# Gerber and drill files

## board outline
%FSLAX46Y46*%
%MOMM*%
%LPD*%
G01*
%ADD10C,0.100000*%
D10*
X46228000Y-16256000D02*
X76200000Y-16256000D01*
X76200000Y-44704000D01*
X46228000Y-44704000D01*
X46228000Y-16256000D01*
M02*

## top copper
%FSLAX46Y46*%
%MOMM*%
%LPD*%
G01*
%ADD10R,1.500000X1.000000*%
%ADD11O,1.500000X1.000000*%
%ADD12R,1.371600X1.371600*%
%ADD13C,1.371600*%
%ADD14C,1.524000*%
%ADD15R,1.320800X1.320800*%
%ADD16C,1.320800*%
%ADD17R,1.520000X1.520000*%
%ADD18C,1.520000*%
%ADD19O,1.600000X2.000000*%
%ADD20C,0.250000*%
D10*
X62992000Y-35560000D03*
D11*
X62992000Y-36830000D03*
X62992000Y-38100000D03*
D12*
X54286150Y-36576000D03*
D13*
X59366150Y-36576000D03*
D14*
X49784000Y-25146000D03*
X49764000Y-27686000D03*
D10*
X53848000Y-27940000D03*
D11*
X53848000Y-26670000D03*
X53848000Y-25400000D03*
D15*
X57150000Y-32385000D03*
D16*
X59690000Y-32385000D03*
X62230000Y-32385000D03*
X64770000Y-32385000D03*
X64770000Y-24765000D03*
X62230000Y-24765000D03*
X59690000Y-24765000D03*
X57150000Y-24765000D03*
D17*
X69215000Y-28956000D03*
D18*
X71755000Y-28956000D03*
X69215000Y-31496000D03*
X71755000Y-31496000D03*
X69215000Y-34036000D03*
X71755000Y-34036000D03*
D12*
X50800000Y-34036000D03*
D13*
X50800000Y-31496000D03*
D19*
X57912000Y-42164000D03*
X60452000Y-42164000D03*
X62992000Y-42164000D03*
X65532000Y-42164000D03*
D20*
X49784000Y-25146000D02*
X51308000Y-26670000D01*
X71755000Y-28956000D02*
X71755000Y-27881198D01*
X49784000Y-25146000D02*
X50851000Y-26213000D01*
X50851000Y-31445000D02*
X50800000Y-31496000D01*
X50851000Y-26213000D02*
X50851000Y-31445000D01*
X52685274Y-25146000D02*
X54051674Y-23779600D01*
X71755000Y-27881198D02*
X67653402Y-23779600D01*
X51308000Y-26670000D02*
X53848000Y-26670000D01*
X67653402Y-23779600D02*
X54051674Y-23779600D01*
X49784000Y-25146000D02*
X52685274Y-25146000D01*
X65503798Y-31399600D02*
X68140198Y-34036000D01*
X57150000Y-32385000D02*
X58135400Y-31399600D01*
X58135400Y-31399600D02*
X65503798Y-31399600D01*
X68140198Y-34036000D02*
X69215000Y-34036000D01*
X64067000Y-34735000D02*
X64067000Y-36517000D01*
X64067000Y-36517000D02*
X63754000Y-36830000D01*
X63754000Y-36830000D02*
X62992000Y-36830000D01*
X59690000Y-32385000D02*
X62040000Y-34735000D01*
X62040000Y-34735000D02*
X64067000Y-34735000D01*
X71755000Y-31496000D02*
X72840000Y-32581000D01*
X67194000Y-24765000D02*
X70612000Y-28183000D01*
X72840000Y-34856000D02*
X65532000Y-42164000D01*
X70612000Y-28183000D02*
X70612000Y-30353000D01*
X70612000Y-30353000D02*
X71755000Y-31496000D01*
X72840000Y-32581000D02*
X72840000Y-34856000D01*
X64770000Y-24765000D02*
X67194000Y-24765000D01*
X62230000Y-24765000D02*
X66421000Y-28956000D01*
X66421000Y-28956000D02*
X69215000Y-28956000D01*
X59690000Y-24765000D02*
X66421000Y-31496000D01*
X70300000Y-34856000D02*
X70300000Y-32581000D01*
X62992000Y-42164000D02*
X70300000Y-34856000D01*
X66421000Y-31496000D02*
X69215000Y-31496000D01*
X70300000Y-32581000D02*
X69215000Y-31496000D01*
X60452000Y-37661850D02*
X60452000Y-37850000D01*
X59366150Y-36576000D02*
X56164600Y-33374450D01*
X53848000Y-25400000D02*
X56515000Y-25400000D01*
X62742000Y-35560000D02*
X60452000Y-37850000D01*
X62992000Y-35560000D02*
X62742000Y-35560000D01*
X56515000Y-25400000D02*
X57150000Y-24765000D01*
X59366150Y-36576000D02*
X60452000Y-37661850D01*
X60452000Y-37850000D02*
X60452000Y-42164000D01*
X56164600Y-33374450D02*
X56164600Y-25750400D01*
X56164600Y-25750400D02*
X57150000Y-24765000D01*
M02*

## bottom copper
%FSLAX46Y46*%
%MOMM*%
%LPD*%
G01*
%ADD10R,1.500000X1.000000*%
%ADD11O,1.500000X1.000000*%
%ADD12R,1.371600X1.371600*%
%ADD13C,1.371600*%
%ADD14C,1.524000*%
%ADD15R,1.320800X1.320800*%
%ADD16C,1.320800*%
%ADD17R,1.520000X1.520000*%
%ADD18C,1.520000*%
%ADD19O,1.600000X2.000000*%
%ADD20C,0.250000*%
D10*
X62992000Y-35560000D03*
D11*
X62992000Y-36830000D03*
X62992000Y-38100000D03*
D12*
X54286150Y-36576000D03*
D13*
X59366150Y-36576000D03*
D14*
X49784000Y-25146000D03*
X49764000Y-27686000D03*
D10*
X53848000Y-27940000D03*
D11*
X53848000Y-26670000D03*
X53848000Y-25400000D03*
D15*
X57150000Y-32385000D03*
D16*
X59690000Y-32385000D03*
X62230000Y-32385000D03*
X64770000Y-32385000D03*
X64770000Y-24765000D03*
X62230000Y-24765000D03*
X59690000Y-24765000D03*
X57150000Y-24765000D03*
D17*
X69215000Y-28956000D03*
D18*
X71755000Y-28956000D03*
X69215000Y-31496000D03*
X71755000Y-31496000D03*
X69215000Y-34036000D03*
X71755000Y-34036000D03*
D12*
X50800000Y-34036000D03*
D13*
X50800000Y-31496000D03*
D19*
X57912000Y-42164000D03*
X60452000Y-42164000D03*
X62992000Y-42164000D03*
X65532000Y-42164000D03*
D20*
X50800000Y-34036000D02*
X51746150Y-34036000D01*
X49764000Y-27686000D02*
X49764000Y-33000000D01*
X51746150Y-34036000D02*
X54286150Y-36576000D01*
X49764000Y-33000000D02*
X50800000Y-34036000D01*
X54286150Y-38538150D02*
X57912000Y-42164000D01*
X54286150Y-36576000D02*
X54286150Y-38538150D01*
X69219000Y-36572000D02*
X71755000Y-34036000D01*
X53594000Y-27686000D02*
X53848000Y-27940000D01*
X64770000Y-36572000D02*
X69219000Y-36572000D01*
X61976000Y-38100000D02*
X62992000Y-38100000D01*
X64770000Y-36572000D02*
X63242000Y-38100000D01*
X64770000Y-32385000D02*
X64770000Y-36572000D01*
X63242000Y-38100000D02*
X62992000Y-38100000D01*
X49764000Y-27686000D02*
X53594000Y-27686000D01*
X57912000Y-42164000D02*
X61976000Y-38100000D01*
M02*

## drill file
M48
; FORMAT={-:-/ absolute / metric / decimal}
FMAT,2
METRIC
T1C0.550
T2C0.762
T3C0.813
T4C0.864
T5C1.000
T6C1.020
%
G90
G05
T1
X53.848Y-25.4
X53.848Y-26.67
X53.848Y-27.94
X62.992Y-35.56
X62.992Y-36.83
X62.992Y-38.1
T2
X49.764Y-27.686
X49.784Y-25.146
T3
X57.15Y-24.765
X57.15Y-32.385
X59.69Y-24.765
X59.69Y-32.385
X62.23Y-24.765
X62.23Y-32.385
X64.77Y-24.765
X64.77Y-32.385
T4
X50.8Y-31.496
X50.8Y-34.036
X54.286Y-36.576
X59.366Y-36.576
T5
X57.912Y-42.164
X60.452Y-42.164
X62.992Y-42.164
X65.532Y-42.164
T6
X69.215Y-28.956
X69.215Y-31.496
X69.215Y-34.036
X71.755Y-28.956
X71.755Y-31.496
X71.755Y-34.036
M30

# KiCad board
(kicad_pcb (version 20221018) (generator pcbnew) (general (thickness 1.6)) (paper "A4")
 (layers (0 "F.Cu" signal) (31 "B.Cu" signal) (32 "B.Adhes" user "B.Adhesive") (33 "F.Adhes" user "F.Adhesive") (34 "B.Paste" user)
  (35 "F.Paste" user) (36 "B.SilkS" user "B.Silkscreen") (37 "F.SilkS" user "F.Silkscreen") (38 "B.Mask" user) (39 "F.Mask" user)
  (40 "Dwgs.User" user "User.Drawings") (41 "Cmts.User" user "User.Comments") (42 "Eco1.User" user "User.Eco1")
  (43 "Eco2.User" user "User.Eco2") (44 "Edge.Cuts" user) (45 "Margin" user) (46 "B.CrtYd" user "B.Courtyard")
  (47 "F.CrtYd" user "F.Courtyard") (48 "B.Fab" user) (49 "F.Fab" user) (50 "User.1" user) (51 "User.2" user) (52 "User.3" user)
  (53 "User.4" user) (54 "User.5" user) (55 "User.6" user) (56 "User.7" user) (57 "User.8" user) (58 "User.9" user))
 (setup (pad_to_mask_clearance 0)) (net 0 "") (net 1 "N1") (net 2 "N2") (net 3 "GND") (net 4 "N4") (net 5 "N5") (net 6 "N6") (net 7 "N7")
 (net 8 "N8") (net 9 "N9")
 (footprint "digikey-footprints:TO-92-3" (layer "F.Cu") (at 62.992 35.56 -90)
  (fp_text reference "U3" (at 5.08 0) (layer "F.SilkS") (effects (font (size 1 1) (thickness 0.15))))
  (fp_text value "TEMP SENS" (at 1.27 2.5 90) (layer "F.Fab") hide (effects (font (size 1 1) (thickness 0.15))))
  (pad "1" thru_hole rect (at 0 0 90) (size 1 1.5) (drill 0.55) (layers "*.Cu" "*.Mask") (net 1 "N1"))
  (pad "2" thru_hole oval (at 1.27 0 90) (size 1 1.5) (drill 0.55) (layers "*.Cu" "*.Mask") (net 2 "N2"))
  (pad "3" thru_hole oval (at 2.54 0 90) (size 1 1.5) (drill 0.55) (layers "*.Cu" "*.Mask") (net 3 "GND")))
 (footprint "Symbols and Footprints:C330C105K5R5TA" (layer "F.Cu") (at 54.28615 36.576)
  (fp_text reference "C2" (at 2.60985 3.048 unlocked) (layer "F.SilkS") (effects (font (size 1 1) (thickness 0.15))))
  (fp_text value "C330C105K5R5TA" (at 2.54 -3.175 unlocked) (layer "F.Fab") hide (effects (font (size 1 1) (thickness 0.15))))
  (pad "1" thru_hole rect (at 0 0) (size 1.3716 1.3716) (drill 0.8636) (layers "*.Cu" "*.Mask") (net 3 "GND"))
  (pad "2" thru_hole circle (at 5.08 0) (size 1.3716 1.3716) (drill 0.8636) (layers "*.Cu" "*.Mask") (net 1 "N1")))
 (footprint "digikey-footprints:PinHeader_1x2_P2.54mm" (layer "F.Cu") (at 49.784 25.146 -90)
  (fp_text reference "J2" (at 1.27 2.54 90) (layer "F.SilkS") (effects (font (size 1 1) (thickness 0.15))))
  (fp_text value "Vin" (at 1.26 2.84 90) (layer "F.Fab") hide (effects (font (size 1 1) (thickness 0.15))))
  (pad "1" thru_hole circle (at 0 0 270) (size 1.524 1.524) (drill 0.762) (layers "*.Cu" "*.Mask") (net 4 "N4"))
  (pad "2" thru_hole circle (at 2.54 0.02 270) (size 1.524 1.524) (drill 0.762) (layers "*.Cu" "*.Mask") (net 3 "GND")))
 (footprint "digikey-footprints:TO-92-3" (layer "F.Cu") (at 53.848 27.94 90)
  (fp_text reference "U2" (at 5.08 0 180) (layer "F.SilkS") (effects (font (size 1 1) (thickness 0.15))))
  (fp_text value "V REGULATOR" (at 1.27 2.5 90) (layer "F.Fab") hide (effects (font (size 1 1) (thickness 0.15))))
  (pad "1" thru_hole rect (at 0 0 270) (size 1 1.5) (drill 0.55) (layers "*.Cu" "*.Mask") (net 3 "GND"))
  (pad "2" thru_hole oval (at 1.27 0 270) (size 1 1.5) (drill 0.55) (layers "*.Cu" "*.Mask") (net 4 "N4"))
  (pad "3" thru_hole oval (at 2.54 0 270) (size 1 1.5) (drill 0.55) (layers "*.Cu" "*.Mask") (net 1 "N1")))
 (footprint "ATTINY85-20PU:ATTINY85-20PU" (layer "F.Cu") (at 60.96 28.575 90)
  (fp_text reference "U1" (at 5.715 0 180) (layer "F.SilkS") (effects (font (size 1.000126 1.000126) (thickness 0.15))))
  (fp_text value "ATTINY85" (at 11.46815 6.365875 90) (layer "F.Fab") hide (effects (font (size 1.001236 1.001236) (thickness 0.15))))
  (pad "1" thru_hole rect (at -3.81 -3.81 90) (size 1.3208 1.3208) (drill 0.8128) (layers "*.Cu" "*.Mask") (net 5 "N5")
   (solder_mask_margin 0.102))
  (pad "2" thru_hole circle (at -3.81 -1.27 90) (size 1.3208 1.3208) (drill 0.8128) (layers "*.Cu" "*.Mask") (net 2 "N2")
   (solder_mask_margin 0.102))
  (pad "3" thru_hole circle (at -3.81 1.27 90) (size 1.3208 1.3208) (drill 0.8128) (layers "*.Cu" "*.Mask") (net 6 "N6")
   (solder_mask_margin 0.102))
  (pad "4" thru_hole circle (at -3.81 3.81 90) (size 1.3208 1.3208) (drill 0.8128) (layers "*.Cu" "*.Mask") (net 3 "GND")
   (solder_mask_margin 0.102))
  (pad "5" thru_hole circle (at 3.81 3.81 90) (size 1.3208 1.3208) (drill 0.8128) (layers "*.Cu" "*.Mask") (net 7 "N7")
   (solder_mask_margin 0.102))
  (pad "6" thru_hole circle (at 3.81 1.27 90) (size 1.3208 1.3208) (drill 0.8128) (layers "*.Cu" "*.Mask") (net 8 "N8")
   (solder_mask_margin 0.102))
  (pad "7" thru_hole circle (at 3.81 -1.27 90) (size 1.3208 1.3208) (drill 0.8128) (layers "*.Cu" "*.Mask") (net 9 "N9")
   (solder_mask_margin 0.102))
  (pad "8" thru_hole circle (at 3.81 -3.81 90) (size 1.3208 1.3208) (drill 0.8128) (layers "*.Cu" "*.Mask") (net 1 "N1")
   (solder_mask_margin 0.102)))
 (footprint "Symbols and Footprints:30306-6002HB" (layer "F.Cu") (at 69.215 28.956)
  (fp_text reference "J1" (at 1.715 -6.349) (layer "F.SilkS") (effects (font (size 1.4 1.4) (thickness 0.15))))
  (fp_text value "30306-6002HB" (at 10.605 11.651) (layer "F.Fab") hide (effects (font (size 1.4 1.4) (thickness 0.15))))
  (pad "1" thru_hole rect (at 0 0) (size 1.52 1.52) (drill 1.02) (layers "*.Cu" "*.Mask") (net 8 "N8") (solder_mask_margin 0.102))
  (pad "2" thru_hole circle (at 2.54 0) (size 1.52 1.52) (drill 1.02) (layers "*.Cu" "*.Mask") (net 4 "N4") (solder_mask_margin 0.102))
  (pad "3" thru_hole circle (at 0 2.54) (size 1.52 1.52) (drill 1.02) (layers "*.Cu" "*.Mask") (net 9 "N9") (solder_mask_margin 0.102))
  (pad "4" thru_hole circle (at 2.54 2.54) (size 1.52 1.52) (drill 1.02) (layers "*.Cu" "*.Mask") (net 7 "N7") (solder_mask_margin 0.102))
  (pad "5" thru_hole circle (at 0 5.08) (size 1.52 1.52) (drill 1.02) (layers "*.Cu" "*.Mask") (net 5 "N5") (solder_mask_margin 0.102))
  (pad "6" thru_hole circle (at 2.54 5.08) (size 1.52 1.52) (drill 1.02) (layers "*.Cu" "*.Mask") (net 3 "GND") (solder_mask_margin 0.102)))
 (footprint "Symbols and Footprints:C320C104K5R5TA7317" (layer "F.Cu") (at 50.8 34.036 90)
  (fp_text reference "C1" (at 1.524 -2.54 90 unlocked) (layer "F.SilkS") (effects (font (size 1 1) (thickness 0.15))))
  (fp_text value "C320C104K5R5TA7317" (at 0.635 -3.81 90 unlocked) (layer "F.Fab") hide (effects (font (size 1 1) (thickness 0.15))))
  (pad "1" thru_hole rect (at 0 0 90) (size 1.3716 1.3716) (drill 0.8636) (layers "*.Cu" "*.Mask") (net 3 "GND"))
  (pad "2" thru_hole circle (at 2.54 0 90) (size 1.3716 1.3716) (drill 0.8636) (layers "*.Cu" "*.Mask") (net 4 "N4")))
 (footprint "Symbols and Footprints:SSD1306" (layer "B.Cu") (at 61.532 31.564)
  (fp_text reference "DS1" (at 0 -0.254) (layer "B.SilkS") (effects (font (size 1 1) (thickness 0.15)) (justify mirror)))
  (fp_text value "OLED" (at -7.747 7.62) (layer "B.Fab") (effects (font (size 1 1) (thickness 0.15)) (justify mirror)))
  (pad "1" thru_hole oval (at -3.62 10.6 270) (size 2 1.6) (drill 1) (layers "*.Cu" "*.Mask") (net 3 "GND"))
  (pad "2" thru_hole oval (at -1.08 10.6 270) (size 2 1.6) (drill 1) (layers "*.Cu" "*.Mask") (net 1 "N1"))
  (pad "3" thru_hole oval (at 1.46 10.6 270) (size 2 1.6) (drill 1) (layers "*.Cu" "*.Mask") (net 9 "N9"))
  (pad "4" thru_hole oval (at 4 10.6 270) (size 2 1.6) (drill 1) (layers "*.Cu" "*.Mask") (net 7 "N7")))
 (gr_rect (start 46.228 16.256) (end 76.2 44.704) (stroke (width 0.1) (type default)) (fill none) (layer "Edge.Cuts"))
 (segment (start 49.784 25.146) (end 51.308 26.67) (width 0.25) (layer "F.Cu") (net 4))
 (segment (start 71.755 28.956) (end 71.755 27.881198) (width 0.25) (layer "F.Cu") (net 4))
 (segment (start 49.784 25.146) (end 50.851 26.213) (width 0.25) (layer "F.Cu") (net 4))
 (segment (start 50.851 31.445) (end 50.8 31.496) (width 0.25) (layer "F.Cu") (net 4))
 (segment (start 50.851 26.213) (end 50.851 31.445) (width 0.25) (layer "F.Cu") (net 4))
 (segment (start 52.685274 25.146) (end 54.051674 23.7796) (width 0.25) (layer "F.Cu") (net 4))
 (segment (start 71.755 27.881198) (end 67.653402 23.7796) (width 0.25) (layer "F.Cu") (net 4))
 (segment (start 51.308 26.67) (end 53.848 26.67) (width 0.25) (layer "F.Cu") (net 4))
 (segment (start 67.653402 23.7796) (end 54.051674 23.7796) (width 0.25) (layer "F.Cu") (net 4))
 (segment (start 49.784 25.146) (end 52.685274 25.146) (width 0.25) (layer "F.Cu") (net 4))
 (segment (start 50.8 34.036) (end 51.74615 34.036) (width 0.25) (layer "B.Cu") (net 3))
 (segment (start 49.764 27.686) (end 49.764 33) (width 0.25) (layer "B.Cu") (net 3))
 (segment (start 51.74615 34.036) (end 54.28615 36.576) (width 0.25) (layer "B.Cu") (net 3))
 (segment (start 49.764 33) (end 50.8 34.036) (width 0.25) (layer "B.Cu") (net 3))
 (segment (start 54.28615 38.53815) (end 57.912 42.164) (width 0.25) (layer "B.Cu") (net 3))
 (segment (start 54.28615 36.576) (end 54.28615 38.53815) (width 0.25) (layer "B.Cu") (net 3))
 (segment (start 69.219 36.572) (end 71.755 34.036) (width 0.25) (layer "B.Cu") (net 3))
 (segment (start 53.594 27.686) (end 53.848 27.94) (width 0.25) (layer "B.Cu") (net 3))
 (segment (start 64.77 36.572) (end 69.219 36.572) (width 0.25) (layer "B.Cu") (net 3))
 (segment (start 61.976 38.1) (end 62.992 38.1) (width 0.25) (layer "B.Cu") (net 3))
 (segment (start 64.77 36.572) (end 63.242 38.1) (width 0.25) (layer "B.Cu") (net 3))
 (segment (start 64.77 32.385) (end 64.77 36.572) (width 0.25) (layer "B.Cu") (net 3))
 (segment (start 63.242 38.1) (end 62.992 38.1) (width 0.25) (layer "B.Cu") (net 3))
 (segment (start 49.764 27.686) (end 53.594 27.686) (width 0.25) (layer "B.Cu") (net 3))
 (segment (start 57.912 42.164) (end 61.976 38.1) (width 0.25) (layer "B.Cu") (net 3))
 (segment (start 65.503798 31.3996) (end 68.140198 34.036) (width 0.25) (layer "F.Cu") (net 5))
 (segment (start 57.15 32.385) (end 58.1354 31.3996) (width 0.25) (layer "F.Cu") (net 5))
 (segment (start 58.1354 31.3996) (end 65.503798 31.3996) (width 0.25) (layer "F.Cu") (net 5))
 (segment (start 68.140198 34.036) (end 69.215 34.036) (width 0.25) (layer "F.Cu") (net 5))
 (segment (start 64.067 34.735) (end 64.067 36.517) (width 0.25) (layer "F.Cu") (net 2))
 (segment (start 64.067 36.517) (end 63.754 36.83) (width 0.25) (layer "F.Cu") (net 2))
 (segment (start 63.754 36.83) (end 62.992 36.83) (width 0.25) (layer "F.Cu") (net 2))
 (segment (start 59.69 32.385) (end 62.04 34.735) (width 0.25) (layer "F.Cu") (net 2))
 (segment (start 62.04 34.735) (end 64.067 34.735) (width 0.25) (layer "F.Cu") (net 2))
 (segment (start 71.755 31.496) (end 72.84 32.581) (width 0.25) (layer "F.Cu") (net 7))
 (segment (start 67.194 24.765) (end 70.612 28.183) (width 0.25) (layer "F.Cu") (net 7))
 (segment (start 72.84 34.856) (end 65.532 42.164) (width 0.25) (layer "F.Cu") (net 7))
 (segment (start 70.612 28.183) (end 70.612 30.353) (width 0.25) (layer "F.Cu") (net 7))
 (segment (start 70.612 30.353) (end 71.755 31.496) (width 0.25) (layer "F.Cu") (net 7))
 (segment (start 72.84 32.581) (end 72.84 34.856) (width 0.25) (layer "F.Cu") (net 7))
 (segment (start 64.77 24.765) (end 67.194 24.765) (width 0.25) (layer "F.Cu") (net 7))
 (segment (start 62.23 24.765) (end 66.421 28.956) (width 0.25) (layer "F.Cu") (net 8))
 (segment (start 66.421 28.956) (end 69.215 28.956) (width 0.25) (layer "F.Cu") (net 8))
 (segment (start 59.69 24.765) (end 66.421 31.496) (width 0.25) (layer "F.Cu") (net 9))
 (segment (start 70.3 34.856) (end 70.3 32.581) (width 0.25) (layer "F.Cu") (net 9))
 (segment (start 62.992 42.164) (end 70.3 34.856) (width 0.25) (layer "F.Cu") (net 9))
 (segment (start 66.421 31.496) (end 69.215 31.496) (width 0.25) (layer "F.Cu") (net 9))
 (segment (start 70.3 32.581) (end 69.215 31.496) (width 0.25) (layer "F.Cu") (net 9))
 (segment (start 60.452 37.66185) (end 60.452 37.85) (width 0.25) (layer "F.Cu") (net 1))
 (segment (start 59.36615 36.576) (end 56.1646 33.37445) (width 0.25) (layer "F.Cu") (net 1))
 (segment (start 53.848 25.4) (end 56.515 25.4) (width 0.25) (layer "F.Cu") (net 1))
 (segment (start 62.742 35.56) (end 60.452 37.85) (width 0.25) (layer "F.Cu") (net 1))
 (segment (start 62.992 35.56) (end 62.742 35.56) (width 0.25) (layer "F.Cu") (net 1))
 (segment (start 56.515 25.4) (end 57.15 24.765) (width 0.25) (layer "F.Cu") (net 1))
 (segment (start 59.36615 36.576) (end 60.452 37.66185) (width 0.25) (layer "F.Cu") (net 1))
 (segment (start 60.452 37.85) (end 60.452 42.164) (width 0.25) (layer "F.Cu") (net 1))
 (segment (start 56.1646 33.37445) (end 56.1646 25.7504) (width 0.25) (layer "F.Cu") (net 1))
 (segment (start 56.1646 25.7504) (end 57.15 24.765) (width 0.25) (layer "F.Cu") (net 1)))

